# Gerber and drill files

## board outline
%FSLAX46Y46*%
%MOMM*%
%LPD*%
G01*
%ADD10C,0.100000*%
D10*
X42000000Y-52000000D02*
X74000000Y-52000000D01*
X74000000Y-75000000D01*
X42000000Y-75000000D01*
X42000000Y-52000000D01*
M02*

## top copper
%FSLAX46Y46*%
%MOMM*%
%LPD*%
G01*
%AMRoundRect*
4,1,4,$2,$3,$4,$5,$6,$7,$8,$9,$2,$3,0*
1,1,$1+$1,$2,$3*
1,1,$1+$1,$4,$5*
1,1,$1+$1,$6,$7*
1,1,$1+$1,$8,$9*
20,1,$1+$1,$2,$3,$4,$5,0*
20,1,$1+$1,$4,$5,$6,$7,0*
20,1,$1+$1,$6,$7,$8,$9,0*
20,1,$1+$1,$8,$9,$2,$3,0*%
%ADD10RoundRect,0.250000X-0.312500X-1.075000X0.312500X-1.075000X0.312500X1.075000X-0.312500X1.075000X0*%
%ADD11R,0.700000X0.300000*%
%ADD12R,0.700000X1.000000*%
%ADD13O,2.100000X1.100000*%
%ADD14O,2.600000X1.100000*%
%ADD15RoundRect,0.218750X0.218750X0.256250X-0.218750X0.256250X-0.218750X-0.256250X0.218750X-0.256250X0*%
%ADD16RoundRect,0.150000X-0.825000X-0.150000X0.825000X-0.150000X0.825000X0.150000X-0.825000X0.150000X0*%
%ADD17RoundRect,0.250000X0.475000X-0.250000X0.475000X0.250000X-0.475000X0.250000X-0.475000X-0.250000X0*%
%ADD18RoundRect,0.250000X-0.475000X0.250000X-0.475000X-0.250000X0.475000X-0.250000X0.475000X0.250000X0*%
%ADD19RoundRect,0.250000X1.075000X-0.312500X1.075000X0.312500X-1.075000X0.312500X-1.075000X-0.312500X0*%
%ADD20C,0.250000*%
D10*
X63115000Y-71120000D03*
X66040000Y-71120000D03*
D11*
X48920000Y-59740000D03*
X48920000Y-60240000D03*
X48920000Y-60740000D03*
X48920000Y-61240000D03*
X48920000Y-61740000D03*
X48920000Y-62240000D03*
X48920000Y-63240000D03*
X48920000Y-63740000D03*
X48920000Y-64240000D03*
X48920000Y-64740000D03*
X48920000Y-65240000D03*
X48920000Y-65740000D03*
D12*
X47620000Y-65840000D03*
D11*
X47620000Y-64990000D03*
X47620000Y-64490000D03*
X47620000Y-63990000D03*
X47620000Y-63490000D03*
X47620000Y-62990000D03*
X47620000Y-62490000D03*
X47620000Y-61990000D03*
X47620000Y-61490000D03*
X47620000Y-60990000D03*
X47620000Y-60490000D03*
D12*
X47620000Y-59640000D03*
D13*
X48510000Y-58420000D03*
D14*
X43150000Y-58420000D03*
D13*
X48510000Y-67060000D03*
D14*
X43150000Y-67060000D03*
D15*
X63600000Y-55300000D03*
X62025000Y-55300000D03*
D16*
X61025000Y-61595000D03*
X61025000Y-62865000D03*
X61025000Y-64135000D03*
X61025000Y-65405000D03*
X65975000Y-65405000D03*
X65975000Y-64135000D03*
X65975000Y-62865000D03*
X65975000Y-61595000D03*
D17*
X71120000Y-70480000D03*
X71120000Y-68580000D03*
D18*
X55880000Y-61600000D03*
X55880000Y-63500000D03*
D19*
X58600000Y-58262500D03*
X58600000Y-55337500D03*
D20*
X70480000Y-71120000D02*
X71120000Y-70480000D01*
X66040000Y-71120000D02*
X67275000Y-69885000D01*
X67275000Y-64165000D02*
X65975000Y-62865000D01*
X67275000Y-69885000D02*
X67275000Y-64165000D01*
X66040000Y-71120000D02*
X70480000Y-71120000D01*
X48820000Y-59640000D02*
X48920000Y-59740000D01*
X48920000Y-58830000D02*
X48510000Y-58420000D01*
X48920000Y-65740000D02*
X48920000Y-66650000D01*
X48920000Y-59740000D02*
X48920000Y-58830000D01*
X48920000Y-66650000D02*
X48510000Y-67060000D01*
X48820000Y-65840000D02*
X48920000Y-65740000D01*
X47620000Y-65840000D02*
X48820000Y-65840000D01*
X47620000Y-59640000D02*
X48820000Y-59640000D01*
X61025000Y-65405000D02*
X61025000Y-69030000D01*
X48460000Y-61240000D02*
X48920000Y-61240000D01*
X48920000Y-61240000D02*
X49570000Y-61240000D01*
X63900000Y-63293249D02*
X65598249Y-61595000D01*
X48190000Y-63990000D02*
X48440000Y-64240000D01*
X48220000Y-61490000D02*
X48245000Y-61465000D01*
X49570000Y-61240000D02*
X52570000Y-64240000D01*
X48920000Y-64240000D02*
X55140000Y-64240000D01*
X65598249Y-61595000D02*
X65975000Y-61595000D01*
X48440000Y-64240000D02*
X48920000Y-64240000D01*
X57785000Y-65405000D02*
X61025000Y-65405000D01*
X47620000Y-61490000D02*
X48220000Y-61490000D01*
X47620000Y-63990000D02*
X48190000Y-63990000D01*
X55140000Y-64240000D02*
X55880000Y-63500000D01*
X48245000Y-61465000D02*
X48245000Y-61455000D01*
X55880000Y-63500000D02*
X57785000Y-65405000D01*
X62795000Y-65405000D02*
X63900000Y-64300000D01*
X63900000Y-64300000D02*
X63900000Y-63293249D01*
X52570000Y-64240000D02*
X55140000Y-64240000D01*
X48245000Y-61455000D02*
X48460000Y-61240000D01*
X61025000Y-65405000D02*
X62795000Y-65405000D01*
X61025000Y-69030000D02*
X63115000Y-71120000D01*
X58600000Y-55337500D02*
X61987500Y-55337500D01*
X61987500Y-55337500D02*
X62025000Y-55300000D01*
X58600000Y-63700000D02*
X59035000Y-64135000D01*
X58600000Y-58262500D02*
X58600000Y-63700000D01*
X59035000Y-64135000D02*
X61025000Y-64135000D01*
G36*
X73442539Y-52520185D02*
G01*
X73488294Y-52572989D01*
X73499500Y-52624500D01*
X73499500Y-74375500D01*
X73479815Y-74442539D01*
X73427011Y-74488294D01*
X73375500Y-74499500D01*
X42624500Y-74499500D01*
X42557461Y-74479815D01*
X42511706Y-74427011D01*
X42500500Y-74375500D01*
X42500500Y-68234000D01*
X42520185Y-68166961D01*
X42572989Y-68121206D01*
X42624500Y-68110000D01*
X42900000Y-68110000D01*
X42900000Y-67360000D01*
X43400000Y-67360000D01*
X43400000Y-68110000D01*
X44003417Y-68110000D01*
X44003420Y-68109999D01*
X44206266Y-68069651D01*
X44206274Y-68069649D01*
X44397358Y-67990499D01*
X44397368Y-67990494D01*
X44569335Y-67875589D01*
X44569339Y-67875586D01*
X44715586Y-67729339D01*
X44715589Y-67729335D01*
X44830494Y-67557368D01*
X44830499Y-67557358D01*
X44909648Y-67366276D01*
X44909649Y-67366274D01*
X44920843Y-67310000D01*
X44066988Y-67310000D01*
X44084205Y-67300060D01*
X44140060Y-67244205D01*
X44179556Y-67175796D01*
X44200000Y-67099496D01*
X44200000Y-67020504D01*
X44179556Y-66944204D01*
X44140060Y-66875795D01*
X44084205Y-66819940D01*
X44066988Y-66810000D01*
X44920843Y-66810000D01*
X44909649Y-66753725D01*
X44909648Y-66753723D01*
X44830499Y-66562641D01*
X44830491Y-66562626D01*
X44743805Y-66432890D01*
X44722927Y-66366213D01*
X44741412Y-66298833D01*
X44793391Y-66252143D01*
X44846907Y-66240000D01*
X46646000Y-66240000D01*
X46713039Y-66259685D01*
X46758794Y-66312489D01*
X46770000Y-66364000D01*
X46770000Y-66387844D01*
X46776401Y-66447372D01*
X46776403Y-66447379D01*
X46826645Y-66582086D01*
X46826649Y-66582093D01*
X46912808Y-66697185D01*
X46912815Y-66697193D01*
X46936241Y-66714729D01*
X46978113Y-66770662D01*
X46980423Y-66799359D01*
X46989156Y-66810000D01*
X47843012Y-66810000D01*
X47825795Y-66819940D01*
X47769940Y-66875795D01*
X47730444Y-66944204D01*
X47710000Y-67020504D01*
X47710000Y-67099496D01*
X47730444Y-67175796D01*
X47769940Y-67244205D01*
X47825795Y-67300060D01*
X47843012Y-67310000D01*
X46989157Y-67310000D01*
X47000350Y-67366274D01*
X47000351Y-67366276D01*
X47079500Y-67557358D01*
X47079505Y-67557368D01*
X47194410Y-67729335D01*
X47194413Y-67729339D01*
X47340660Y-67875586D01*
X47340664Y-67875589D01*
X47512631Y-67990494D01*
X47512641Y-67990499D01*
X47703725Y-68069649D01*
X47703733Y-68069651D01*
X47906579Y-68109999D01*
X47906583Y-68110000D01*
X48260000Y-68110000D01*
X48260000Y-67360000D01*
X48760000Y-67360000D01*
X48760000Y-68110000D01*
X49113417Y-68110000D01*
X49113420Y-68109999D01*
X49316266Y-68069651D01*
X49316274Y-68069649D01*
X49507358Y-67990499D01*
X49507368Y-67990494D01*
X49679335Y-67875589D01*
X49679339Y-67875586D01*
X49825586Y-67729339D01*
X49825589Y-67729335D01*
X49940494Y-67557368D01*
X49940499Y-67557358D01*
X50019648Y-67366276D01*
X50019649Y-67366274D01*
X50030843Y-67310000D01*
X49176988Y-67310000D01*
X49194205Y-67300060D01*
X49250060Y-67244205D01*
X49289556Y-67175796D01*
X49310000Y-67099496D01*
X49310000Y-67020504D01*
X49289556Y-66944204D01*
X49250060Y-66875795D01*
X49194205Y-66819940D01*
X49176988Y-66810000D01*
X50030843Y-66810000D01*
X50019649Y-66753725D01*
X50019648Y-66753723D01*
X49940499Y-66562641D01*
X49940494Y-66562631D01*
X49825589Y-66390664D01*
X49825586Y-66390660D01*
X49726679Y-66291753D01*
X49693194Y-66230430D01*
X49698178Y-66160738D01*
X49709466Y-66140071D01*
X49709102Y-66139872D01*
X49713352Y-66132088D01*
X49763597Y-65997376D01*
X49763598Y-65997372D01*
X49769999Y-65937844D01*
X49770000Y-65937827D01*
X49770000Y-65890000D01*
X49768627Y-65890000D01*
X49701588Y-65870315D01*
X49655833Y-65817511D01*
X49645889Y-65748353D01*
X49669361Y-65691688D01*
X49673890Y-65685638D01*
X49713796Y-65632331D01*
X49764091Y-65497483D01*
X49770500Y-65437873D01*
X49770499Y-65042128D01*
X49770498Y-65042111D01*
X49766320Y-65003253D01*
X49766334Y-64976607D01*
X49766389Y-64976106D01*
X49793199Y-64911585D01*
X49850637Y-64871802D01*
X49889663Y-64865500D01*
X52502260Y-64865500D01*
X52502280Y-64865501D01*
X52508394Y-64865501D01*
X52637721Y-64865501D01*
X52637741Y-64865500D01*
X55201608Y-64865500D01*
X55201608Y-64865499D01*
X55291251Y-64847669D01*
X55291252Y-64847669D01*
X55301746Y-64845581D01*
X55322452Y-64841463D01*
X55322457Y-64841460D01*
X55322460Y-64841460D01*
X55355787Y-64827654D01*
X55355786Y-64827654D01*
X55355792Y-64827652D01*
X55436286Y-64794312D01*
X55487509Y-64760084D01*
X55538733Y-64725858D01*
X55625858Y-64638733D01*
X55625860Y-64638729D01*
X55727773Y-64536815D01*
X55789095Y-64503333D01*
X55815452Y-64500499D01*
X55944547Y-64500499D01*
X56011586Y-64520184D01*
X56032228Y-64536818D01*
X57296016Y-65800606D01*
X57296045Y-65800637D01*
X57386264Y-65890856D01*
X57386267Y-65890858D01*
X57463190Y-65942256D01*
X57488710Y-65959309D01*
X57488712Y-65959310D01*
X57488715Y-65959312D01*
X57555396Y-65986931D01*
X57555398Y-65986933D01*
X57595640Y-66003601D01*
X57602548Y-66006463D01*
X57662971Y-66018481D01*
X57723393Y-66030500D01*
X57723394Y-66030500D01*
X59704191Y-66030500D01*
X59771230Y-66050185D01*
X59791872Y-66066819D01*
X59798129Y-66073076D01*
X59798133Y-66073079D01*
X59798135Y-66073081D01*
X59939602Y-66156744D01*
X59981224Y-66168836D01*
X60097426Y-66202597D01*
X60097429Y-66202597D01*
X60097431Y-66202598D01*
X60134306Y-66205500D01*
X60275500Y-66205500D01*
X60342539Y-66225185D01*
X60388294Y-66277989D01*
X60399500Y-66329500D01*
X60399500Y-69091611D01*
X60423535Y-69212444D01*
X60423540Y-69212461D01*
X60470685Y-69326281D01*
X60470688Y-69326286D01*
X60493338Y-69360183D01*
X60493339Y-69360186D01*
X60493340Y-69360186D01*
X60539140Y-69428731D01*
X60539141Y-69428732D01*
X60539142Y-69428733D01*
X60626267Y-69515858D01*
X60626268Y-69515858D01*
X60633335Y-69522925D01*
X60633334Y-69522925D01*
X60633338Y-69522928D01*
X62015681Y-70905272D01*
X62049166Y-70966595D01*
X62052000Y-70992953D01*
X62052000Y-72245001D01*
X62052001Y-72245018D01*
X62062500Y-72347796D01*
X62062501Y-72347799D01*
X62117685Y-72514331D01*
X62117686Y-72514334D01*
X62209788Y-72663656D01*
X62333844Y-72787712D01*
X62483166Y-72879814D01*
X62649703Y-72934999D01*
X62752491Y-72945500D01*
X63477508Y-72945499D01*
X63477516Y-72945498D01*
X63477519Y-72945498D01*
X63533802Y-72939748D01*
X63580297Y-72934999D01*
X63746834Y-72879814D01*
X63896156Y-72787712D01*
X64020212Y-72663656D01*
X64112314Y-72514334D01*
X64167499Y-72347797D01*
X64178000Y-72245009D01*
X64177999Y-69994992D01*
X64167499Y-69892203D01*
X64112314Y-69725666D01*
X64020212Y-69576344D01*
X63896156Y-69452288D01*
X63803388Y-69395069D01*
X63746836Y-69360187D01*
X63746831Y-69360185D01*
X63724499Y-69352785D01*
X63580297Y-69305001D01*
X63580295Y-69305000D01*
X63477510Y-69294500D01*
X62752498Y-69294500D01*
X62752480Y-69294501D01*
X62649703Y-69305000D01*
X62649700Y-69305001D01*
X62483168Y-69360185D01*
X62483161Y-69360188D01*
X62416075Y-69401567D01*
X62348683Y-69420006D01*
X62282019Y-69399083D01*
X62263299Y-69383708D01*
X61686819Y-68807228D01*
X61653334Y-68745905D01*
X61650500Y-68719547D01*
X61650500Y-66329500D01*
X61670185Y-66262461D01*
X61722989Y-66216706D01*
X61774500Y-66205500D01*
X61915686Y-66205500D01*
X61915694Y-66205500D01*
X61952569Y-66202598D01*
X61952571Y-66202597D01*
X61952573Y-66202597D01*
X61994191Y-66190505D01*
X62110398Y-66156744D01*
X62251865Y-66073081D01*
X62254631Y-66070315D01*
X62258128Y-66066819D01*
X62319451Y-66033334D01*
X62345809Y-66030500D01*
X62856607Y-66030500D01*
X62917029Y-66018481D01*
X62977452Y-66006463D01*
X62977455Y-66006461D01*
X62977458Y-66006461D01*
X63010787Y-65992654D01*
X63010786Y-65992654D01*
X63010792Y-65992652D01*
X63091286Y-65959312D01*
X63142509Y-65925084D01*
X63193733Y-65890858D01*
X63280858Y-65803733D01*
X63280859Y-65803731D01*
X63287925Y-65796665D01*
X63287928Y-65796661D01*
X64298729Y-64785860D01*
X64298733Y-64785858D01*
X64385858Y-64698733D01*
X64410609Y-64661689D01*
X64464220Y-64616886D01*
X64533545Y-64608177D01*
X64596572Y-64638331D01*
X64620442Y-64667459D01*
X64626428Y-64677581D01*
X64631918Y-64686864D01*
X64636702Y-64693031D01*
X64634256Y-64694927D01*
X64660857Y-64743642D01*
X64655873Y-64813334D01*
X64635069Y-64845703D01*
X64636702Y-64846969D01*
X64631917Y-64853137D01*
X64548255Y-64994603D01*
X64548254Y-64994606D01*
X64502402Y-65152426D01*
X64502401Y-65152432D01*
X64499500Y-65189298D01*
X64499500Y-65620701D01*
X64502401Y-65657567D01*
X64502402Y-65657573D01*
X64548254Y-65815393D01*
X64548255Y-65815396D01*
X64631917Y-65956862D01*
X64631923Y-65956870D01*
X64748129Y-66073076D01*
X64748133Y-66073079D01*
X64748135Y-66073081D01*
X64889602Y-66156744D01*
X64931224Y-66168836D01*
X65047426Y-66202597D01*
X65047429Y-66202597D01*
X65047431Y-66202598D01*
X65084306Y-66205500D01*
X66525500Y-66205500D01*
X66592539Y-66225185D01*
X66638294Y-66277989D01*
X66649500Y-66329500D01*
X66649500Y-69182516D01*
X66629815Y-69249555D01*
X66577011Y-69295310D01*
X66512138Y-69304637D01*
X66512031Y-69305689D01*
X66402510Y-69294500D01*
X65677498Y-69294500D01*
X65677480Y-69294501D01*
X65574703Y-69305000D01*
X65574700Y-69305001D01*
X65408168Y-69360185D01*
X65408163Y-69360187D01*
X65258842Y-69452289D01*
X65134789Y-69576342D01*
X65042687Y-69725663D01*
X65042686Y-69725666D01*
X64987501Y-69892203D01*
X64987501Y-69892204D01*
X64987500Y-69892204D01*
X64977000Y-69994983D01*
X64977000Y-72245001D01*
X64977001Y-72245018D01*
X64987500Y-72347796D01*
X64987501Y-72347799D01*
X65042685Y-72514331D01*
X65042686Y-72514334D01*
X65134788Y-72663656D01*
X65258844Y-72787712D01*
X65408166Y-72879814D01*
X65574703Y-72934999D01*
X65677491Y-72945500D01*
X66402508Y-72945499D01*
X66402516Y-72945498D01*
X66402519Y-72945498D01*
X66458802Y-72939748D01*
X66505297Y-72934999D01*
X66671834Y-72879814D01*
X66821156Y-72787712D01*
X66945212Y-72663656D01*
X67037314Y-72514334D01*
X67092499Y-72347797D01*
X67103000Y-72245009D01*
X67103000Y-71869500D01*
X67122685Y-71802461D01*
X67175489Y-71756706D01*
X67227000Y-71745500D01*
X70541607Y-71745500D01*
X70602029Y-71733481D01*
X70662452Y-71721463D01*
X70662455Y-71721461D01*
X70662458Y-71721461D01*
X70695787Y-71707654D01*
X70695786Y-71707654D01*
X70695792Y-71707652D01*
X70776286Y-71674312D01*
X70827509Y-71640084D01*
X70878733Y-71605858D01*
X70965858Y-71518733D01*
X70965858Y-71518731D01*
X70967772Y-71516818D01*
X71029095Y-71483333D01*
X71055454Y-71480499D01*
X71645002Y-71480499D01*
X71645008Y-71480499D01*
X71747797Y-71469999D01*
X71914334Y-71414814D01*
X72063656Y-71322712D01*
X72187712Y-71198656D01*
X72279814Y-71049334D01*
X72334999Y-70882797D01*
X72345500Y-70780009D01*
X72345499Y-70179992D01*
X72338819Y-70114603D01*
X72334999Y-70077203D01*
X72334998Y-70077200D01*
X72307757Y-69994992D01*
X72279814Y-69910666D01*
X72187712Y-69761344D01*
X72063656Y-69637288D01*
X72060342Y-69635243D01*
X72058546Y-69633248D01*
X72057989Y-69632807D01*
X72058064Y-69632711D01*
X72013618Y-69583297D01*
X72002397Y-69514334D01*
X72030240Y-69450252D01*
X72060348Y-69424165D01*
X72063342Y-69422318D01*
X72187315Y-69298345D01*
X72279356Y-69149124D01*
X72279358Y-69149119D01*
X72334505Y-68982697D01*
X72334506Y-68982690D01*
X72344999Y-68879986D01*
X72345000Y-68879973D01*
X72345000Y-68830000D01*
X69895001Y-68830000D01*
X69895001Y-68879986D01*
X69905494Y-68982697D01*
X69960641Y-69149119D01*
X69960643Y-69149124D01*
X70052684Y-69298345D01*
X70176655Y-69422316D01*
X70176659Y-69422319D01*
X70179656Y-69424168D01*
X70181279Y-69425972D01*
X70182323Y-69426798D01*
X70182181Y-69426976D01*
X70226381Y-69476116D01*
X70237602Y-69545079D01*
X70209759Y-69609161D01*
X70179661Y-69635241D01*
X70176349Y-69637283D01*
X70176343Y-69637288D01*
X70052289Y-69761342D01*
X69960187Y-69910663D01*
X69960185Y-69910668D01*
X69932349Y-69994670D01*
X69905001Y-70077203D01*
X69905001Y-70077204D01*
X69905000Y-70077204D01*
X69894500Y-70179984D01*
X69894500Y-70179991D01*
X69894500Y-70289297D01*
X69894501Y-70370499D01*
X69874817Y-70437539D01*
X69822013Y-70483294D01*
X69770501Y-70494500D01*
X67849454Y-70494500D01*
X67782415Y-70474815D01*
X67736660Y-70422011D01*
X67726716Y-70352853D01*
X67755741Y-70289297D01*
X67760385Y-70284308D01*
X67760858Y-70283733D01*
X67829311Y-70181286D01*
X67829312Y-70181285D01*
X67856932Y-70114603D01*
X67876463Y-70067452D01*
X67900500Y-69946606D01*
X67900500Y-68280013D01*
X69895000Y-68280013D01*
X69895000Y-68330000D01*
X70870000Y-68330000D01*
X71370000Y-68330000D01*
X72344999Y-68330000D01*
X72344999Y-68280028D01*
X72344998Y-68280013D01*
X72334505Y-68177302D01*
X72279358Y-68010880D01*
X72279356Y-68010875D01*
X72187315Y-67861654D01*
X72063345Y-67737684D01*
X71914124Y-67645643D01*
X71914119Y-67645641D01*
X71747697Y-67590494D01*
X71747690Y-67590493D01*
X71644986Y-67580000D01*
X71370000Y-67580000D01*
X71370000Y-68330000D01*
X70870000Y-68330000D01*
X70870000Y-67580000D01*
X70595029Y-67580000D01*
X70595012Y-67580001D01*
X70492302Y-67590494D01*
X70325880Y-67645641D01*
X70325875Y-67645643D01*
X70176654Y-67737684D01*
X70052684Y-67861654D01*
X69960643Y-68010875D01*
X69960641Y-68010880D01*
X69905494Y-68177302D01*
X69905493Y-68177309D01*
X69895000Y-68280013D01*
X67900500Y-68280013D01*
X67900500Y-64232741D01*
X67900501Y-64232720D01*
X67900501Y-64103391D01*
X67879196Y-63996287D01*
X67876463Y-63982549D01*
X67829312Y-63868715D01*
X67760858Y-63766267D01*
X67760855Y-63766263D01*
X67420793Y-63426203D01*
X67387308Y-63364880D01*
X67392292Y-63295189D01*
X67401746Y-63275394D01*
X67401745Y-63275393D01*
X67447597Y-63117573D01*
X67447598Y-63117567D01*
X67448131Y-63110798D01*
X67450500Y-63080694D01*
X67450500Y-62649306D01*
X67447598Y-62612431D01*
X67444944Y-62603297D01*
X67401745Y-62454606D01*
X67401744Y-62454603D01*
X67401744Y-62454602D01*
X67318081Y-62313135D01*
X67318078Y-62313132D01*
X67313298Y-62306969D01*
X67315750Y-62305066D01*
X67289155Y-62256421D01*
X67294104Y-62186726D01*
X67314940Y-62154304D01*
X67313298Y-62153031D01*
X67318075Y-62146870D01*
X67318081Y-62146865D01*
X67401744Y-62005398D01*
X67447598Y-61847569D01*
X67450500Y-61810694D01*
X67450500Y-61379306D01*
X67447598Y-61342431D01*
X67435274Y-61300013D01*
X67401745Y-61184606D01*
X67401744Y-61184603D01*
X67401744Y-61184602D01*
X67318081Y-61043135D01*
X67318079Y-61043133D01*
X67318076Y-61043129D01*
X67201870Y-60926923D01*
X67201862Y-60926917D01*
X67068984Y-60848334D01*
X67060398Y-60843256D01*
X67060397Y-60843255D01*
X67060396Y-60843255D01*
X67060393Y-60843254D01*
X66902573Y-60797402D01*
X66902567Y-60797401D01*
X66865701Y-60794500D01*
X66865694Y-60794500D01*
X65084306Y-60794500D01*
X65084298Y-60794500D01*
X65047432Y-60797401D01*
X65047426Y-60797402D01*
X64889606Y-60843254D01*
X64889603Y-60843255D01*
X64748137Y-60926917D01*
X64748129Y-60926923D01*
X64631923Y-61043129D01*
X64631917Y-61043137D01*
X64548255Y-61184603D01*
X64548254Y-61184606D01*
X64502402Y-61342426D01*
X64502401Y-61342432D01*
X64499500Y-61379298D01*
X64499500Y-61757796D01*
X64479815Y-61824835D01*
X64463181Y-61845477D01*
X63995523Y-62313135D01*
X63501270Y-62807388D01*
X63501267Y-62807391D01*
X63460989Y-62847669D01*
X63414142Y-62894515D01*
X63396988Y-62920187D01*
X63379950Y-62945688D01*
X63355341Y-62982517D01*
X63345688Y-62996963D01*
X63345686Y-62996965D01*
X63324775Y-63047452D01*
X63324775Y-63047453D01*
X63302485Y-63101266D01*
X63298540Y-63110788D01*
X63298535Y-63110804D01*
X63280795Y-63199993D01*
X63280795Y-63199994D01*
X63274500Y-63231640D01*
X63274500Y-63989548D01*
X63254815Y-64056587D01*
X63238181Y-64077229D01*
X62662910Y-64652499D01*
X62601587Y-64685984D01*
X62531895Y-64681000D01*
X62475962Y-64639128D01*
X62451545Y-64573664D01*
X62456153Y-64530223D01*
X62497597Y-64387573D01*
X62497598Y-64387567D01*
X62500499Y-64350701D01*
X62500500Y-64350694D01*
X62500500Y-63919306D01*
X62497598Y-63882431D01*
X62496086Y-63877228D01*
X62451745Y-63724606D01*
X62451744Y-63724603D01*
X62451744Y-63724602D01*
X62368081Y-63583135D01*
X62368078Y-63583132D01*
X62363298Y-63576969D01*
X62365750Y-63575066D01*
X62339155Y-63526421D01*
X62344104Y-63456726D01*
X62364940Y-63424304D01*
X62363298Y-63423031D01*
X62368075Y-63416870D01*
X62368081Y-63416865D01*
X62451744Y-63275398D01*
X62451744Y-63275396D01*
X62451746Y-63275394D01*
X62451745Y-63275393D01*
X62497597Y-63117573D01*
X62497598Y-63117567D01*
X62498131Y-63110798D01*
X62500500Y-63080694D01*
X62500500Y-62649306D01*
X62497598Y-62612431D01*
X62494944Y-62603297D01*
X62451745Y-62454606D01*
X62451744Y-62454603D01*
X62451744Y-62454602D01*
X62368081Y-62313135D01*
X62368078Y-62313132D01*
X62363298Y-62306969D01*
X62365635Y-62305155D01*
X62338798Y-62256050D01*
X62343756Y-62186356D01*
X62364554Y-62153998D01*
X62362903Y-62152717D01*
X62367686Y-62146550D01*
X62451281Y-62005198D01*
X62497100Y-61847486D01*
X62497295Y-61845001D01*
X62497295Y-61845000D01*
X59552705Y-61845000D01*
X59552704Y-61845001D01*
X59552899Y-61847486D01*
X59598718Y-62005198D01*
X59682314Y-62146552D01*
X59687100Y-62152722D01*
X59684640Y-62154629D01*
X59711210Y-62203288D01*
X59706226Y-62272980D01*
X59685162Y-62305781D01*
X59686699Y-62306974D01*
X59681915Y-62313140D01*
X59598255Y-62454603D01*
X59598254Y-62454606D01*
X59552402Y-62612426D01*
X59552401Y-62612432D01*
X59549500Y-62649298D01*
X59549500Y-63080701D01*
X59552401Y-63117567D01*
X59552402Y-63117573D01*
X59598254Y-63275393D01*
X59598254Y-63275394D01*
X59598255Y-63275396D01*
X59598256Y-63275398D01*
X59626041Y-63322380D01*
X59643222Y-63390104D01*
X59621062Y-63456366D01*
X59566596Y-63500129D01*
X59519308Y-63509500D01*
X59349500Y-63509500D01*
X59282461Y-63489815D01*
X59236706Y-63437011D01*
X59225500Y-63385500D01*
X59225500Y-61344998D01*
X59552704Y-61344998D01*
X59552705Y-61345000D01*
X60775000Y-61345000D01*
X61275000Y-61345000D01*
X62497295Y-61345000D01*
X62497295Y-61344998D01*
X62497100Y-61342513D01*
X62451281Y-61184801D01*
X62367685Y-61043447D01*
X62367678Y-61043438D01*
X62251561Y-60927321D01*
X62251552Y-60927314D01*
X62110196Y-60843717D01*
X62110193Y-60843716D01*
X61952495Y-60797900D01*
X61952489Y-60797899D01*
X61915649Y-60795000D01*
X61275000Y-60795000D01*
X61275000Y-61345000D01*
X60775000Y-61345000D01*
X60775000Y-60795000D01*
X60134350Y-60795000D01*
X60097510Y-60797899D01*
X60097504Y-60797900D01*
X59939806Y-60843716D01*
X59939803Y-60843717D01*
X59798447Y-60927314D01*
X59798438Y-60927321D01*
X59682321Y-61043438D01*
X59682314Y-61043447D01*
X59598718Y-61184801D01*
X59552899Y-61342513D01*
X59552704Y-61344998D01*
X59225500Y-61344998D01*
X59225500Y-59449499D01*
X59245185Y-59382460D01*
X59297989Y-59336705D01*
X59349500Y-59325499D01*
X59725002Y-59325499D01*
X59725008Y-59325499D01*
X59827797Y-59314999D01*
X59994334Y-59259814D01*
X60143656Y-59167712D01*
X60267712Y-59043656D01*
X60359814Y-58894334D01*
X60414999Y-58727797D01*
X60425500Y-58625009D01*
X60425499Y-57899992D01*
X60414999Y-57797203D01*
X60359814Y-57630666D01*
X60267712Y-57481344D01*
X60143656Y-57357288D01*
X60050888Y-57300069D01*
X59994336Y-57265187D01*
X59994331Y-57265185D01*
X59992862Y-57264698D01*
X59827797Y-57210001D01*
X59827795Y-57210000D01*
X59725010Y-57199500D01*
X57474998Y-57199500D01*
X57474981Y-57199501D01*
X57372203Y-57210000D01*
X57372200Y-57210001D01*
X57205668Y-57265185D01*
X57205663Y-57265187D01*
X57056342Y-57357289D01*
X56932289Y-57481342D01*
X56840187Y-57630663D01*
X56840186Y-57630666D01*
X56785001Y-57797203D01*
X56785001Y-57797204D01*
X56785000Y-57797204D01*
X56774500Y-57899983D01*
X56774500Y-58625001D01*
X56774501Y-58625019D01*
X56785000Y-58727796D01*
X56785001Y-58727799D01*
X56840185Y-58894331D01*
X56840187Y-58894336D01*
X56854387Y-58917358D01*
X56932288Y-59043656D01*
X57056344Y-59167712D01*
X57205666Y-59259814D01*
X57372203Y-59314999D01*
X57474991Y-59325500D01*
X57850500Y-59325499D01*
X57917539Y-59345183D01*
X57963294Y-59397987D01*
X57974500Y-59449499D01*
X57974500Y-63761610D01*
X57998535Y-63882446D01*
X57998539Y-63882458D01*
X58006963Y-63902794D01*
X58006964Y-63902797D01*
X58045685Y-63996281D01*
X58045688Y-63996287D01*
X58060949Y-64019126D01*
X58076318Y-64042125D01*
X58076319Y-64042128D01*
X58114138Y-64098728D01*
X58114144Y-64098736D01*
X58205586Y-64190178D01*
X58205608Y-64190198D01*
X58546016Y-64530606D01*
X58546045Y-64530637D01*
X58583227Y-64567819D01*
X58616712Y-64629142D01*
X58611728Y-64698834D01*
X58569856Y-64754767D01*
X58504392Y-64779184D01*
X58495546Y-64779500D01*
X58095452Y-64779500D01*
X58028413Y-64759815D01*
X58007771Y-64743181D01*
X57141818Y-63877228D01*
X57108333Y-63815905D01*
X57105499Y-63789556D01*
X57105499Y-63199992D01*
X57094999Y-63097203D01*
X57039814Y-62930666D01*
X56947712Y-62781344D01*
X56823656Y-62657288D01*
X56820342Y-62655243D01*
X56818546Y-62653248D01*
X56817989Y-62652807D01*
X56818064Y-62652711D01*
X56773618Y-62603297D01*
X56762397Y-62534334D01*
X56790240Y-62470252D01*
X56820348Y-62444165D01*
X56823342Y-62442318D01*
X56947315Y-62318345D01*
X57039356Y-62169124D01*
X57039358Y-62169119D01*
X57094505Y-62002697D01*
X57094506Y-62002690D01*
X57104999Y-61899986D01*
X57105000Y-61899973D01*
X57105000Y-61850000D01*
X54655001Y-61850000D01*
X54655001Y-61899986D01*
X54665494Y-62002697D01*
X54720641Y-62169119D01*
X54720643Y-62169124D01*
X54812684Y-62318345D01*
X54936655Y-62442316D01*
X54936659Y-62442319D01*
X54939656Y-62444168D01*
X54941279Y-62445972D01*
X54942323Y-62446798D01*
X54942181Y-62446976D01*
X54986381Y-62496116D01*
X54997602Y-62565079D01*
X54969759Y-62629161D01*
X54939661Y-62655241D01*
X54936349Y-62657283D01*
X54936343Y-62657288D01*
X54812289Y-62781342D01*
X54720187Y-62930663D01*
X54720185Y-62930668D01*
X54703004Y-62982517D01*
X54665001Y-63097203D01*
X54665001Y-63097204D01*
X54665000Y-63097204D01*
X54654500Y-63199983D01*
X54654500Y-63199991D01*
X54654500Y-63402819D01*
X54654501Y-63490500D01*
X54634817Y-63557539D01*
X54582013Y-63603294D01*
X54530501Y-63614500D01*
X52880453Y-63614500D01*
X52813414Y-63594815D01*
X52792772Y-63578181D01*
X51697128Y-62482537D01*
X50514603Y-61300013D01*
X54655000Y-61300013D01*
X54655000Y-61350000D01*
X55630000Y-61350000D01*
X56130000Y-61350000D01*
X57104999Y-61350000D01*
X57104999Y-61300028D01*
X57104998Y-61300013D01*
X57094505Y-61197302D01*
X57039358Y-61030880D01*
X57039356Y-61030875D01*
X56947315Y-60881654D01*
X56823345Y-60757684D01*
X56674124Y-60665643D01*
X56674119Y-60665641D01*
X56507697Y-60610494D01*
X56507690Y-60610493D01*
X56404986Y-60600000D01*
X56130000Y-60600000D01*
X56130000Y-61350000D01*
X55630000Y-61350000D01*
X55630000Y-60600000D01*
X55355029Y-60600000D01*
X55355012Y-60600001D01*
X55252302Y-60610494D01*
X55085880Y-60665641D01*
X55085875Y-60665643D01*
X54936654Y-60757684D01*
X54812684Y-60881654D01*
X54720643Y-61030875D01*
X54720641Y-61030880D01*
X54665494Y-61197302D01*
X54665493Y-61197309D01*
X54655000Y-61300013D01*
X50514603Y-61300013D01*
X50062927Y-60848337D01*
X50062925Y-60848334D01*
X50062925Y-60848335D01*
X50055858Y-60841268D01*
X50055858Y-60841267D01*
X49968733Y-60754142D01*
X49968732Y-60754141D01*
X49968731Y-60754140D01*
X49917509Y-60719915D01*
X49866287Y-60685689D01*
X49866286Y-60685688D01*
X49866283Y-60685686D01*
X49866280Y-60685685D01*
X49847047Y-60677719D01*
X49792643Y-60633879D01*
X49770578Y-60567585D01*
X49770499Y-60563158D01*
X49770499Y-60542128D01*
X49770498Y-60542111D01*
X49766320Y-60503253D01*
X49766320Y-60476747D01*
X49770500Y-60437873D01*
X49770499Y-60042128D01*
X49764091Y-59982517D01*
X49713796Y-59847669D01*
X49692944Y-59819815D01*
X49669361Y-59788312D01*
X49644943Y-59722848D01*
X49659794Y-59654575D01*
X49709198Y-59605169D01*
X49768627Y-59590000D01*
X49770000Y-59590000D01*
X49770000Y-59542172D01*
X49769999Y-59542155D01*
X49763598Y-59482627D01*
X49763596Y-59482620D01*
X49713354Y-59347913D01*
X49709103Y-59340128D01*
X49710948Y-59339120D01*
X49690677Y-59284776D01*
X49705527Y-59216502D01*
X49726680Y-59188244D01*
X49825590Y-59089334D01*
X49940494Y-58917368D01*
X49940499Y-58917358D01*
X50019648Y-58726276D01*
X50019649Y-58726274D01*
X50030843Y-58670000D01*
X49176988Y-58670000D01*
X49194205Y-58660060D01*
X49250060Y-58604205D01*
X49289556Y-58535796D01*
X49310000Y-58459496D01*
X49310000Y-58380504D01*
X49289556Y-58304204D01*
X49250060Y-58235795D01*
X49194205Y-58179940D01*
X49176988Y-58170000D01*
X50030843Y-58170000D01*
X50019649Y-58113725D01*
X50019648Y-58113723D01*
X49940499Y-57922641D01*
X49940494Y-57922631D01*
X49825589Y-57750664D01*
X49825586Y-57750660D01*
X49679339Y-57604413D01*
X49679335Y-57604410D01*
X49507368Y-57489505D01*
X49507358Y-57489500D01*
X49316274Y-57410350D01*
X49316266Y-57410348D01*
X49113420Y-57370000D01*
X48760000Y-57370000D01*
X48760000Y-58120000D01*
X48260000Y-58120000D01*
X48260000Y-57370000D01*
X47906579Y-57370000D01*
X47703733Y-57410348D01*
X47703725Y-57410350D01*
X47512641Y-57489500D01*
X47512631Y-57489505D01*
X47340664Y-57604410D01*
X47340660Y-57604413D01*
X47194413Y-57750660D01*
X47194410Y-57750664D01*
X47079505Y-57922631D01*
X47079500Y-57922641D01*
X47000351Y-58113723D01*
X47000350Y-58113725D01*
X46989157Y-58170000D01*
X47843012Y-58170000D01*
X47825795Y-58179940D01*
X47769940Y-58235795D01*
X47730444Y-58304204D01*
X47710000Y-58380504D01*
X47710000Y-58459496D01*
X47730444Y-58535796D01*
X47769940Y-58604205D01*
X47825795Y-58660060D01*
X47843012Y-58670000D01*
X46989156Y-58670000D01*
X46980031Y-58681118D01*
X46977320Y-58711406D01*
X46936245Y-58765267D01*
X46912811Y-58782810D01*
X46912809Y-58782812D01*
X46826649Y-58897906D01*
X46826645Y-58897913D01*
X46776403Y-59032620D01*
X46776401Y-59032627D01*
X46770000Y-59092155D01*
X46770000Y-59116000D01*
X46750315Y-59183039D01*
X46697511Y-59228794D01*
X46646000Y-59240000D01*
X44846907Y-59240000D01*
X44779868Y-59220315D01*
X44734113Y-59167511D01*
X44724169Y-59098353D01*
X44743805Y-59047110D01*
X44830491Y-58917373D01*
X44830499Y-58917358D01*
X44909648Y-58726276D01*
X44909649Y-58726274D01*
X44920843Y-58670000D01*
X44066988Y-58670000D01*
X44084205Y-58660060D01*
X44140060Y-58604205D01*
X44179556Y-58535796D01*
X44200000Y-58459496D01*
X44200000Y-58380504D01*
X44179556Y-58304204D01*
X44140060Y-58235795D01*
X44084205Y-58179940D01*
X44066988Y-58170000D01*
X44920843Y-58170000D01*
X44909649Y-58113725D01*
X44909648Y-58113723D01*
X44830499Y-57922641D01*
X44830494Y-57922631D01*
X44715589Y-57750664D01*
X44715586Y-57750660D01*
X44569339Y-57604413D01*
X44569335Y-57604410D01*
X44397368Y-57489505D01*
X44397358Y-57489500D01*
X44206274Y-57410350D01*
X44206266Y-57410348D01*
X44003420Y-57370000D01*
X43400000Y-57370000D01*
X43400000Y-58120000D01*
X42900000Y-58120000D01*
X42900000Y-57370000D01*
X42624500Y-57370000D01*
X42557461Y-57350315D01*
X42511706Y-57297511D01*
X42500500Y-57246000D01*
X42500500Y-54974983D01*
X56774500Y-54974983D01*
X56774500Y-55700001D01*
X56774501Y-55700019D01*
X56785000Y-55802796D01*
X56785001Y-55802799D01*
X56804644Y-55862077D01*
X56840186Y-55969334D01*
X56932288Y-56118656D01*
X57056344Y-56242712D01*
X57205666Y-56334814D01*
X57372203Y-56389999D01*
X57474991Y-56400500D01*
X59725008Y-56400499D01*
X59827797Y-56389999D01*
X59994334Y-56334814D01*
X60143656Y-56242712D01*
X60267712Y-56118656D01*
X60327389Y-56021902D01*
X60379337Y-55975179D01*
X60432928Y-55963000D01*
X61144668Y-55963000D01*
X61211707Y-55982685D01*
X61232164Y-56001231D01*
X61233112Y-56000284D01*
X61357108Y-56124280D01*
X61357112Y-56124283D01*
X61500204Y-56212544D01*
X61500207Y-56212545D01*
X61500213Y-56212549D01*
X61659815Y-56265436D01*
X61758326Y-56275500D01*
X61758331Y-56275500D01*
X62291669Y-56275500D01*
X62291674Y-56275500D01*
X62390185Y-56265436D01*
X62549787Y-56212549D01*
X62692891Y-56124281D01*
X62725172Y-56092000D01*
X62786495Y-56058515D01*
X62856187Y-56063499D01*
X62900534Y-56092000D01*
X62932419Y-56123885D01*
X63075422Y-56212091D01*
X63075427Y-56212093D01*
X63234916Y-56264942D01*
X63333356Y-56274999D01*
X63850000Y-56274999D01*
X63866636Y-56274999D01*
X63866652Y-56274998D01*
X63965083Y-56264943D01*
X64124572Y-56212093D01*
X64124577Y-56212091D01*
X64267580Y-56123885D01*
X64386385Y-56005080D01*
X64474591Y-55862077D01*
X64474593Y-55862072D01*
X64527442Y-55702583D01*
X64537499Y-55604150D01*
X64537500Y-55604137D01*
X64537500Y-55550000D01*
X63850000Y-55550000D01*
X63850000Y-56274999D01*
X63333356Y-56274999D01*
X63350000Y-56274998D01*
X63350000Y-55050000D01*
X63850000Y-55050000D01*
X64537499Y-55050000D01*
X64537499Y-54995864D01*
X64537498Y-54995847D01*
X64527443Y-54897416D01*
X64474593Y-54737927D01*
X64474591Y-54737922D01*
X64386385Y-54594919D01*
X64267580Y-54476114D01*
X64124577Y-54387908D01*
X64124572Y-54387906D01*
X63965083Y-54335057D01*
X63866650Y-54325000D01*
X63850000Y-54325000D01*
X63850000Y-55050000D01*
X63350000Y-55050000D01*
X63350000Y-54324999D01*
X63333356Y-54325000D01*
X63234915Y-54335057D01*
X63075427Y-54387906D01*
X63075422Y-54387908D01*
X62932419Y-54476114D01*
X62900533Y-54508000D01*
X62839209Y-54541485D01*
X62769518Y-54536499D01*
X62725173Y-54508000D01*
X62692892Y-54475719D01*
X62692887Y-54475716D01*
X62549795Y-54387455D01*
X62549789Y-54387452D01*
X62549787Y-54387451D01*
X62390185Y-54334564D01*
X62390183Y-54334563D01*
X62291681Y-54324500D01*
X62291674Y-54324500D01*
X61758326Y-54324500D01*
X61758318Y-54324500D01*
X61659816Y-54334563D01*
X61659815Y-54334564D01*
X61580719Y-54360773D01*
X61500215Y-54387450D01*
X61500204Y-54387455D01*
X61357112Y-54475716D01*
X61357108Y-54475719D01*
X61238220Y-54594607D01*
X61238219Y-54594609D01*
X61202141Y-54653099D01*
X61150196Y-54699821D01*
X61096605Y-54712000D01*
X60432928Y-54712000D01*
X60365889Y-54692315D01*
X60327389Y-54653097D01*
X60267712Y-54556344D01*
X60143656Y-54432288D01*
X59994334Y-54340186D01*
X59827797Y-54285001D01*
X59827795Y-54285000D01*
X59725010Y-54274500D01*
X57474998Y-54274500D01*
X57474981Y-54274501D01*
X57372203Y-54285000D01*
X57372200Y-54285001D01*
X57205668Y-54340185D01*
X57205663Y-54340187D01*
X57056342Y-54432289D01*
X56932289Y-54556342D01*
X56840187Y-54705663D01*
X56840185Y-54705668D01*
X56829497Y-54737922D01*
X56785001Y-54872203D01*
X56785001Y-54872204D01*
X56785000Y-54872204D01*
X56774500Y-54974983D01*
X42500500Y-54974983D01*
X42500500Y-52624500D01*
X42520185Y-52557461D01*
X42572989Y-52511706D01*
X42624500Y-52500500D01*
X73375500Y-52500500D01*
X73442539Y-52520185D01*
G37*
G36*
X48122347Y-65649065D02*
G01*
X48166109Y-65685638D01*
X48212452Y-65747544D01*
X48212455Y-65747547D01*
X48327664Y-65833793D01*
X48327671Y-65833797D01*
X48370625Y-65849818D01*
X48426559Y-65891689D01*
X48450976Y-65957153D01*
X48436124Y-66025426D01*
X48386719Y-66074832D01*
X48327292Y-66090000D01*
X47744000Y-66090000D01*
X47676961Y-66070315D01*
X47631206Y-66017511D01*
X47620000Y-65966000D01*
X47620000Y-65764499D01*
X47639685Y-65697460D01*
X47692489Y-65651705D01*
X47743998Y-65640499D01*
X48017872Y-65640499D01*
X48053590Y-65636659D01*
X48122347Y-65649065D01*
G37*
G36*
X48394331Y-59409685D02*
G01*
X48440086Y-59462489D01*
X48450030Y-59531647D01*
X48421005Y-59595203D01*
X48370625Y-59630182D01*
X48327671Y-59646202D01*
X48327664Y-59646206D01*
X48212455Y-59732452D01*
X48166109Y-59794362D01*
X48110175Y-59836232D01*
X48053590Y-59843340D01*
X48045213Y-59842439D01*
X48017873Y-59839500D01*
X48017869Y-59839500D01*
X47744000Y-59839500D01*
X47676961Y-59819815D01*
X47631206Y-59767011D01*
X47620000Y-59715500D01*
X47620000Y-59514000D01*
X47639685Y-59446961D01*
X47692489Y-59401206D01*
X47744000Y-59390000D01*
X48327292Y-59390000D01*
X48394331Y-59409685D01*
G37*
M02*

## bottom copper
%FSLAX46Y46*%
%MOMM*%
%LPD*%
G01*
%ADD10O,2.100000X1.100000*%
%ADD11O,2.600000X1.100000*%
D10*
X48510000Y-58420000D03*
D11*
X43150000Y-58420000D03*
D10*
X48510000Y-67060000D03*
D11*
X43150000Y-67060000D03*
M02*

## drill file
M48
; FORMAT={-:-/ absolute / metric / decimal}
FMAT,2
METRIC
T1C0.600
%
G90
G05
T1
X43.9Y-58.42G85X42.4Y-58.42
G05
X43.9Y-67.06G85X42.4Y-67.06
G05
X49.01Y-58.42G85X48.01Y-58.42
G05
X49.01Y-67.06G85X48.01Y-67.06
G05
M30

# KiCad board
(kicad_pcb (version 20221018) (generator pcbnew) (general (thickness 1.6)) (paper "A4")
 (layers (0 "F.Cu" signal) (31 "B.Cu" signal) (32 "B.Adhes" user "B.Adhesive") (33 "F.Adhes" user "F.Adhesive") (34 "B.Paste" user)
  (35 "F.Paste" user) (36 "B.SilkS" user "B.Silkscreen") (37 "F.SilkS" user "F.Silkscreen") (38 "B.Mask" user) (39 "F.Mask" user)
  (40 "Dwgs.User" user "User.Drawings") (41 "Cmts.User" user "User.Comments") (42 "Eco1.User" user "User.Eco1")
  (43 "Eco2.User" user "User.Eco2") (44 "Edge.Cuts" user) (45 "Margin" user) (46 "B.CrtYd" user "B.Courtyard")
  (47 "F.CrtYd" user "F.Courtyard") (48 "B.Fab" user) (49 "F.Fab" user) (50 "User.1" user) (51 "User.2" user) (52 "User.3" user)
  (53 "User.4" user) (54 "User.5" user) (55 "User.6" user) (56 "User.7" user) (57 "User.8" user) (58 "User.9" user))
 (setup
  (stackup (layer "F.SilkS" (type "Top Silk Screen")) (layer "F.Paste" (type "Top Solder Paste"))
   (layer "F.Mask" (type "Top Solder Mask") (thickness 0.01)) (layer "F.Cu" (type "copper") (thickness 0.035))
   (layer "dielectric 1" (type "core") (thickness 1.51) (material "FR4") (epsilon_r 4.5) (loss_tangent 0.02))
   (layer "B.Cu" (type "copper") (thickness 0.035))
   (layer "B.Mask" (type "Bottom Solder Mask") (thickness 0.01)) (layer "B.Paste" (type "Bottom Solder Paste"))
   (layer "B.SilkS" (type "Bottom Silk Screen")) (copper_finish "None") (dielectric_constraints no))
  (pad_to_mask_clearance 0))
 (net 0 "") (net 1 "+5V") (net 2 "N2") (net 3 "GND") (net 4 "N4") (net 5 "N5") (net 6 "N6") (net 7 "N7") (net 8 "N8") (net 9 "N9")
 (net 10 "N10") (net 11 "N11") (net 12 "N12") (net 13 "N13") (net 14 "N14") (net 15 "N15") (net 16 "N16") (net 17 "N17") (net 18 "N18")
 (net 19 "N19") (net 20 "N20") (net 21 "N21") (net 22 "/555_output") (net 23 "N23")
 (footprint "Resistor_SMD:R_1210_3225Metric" (layer "F.Cu") (at 64.5775 71.12)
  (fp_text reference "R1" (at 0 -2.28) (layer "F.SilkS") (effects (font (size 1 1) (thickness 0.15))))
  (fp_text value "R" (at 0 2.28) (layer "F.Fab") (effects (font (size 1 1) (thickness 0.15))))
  (pad "1" smd roundrect (at -1.4625 0) (size 1.125 2.65) (layers "F.Cu" "F.Paste" "F.Mask") (roundrect_rratio 0.222222) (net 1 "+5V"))
  (pad "2" smd roundrect (at 1.4625 0) (size 1.125 2.65) (layers "F.Cu" "F.Paste" "F.Mask") (roundrect_rratio 0.222222) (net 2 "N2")))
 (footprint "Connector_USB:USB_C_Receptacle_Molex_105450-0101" (layer "F.Cu") (at 45.705 62.74 -90)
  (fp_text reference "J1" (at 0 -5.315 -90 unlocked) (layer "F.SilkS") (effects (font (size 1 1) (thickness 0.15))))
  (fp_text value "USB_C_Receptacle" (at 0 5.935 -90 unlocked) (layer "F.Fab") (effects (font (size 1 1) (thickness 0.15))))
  (pad "A1" smd rect (at -3 -3.215 270) (size 0.3 0.7) (layers "F.Cu" "F.Paste" "F.Mask") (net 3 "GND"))
  (pad "A2" smd rect (at -2.5 -3.215 270) (size 0.3 0.7) (layers "F.Cu" "F.Paste" "F.Mask") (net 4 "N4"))
  (pad "A3" smd rect (at -2 -3.215 270) (size 0.3 0.7) (layers "F.Cu" "F.Paste" "F.Mask") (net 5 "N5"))
  (pad "A4" smd rect (at -1.5 -3.215 270) (size 0.3 0.7) (layers "F.Cu" "F.Paste" "F.Mask") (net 1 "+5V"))
  (pad "A5" smd rect (at -1 -3.215 270) (size 0.3 0.7) (layers "F.Cu" "F.Paste" "F.Mask") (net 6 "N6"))
  (pad "A6" smd rect (at -0.5 -3.215 270) (size 0.3 0.7) (layers "F.Cu" "F.Paste" "F.Mask") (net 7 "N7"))
  (pad "A7" smd rect (at 0.5 -3.215 270) (size 0.3 0.7) (layers "F.Cu" "F.Paste" "F.Mask") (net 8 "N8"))
  (pad "A8" smd rect (at 1 -3.215 270) (size 0.3 0.7) (layers "F.Cu" "F.Paste" "F.Mask") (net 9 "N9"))
  (pad "A9" smd rect (at 1.5 -3.215 270) (size 0.3 0.7) (layers "F.Cu" "F.Paste" "F.Mask") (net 1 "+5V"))
  (pad "A10" smd rect (at 2 -3.215 270) (size 0.3 0.7) (layers "F.Cu" "F.Paste" "F.Mask") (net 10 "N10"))
  (pad "A11" smd rect (at 2.5 -3.215 270) (size 0.3 0.7) (layers "F.Cu" "F.Paste" "F.Mask") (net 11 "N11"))
  (pad "A12" smd rect (at 3 -3.215 270) (size 0.3 0.7) (layers "F.Cu" "F.Paste" "F.Mask") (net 3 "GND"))
  (pad "B1" smd rect (at 3.1 -1.915 270) (size 1 0.7) (layers "F.Cu" "F.Paste" "F.Mask") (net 3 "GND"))
  (pad "B2" smd rect (at 2.25 -1.915 270) (size 0.3 0.7) (layers "F.Cu" "F.Paste" "F.Mask") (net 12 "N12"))
  (pad "B3" smd rect (at 1.75 -1.915 270) (size 0.3 0.7) (layers "F.Cu" "F.Paste" "F.Mask") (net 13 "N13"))
  (pad "B4" smd rect (at 1.25 -1.915 270) (size 0.3 0.7) (layers "F.Cu" "F.Paste" "F.Mask") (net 1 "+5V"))
  (pad "B5" smd rect (at 0.75 -1.915 270) (size 0.3 0.7) (layers "F.Cu" "F.Paste" "F.Mask") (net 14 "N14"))
  (pad "B6" smd rect (at 0.25 -1.915 270) (size 0.3 0.7) (layers "F.Cu" "F.Paste" "F.Mask") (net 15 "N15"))
  (pad "B7" smd rect (at -0.25 -1.915 270) (size 0.3 0.7) (layers "F.Cu" "F.Paste" "F.Mask") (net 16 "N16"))
  (pad "B8" smd rect (at -0.75 -1.915 270) (size 0.3 0.7) (layers "F.Cu" "F.Paste" "F.Mask") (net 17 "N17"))
  (pad "B9" smd rect (at -1.25 -1.915 270) (size 0.3 0.7) (layers "F.Cu" "F.Paste" "F.Mask") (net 1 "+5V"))
  (pad "B10" smd rect (at -1.75 -1.915 270) (size 0.3 0.7) (layers "F.Cu" "F.Paste" "F.Mask") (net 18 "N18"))
  (pad "B11" smd rect (at -2.25 -1.915 270) (size 0.3 0.7) (layers "F.Cu" "F.Paste" "F.Mask") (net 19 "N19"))
  (pad "B12" smd rect (at -3.1 -1.915 270) (size 1 0.7) (layers "F.Cu" "F.Paste" "F.Mask") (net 3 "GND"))
  (pad "S1" thru_hole oval (at -4.32 -2.805 270) (size 1.1 2.1) (drill oval 0.6 1.6) (layers "*.Cu" "*.Mask") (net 3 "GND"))
  (pad "S1" thru_hole oval (at -4.32 2.555 270) (size 1.1 2.6) (drill oval 0.6 2.1) (layers "*.Cu" "*.Mask") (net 3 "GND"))
  (pad "S1" thru_hole oval (at 4.32 -2.805 270) (size 1.1 2.1) (drill oval 0.6 1.6) (layers "*.Cu" "*.Mask") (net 3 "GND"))
  (pad "S1" thru_hole oval (at 4.32 2.555 270) (size 1.1 2.6) (drill oval 0.6 2.1) (layers "*.Cu" "*.Mask") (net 3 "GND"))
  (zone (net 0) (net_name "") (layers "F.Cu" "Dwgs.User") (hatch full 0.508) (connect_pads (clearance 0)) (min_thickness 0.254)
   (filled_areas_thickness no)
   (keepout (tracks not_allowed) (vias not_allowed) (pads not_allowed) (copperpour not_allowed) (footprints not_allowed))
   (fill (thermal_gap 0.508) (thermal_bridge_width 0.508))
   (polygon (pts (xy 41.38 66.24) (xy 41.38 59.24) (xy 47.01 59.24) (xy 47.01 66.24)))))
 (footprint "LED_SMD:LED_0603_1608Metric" (layer "F.Cu") (at 62.8125 55.3 180)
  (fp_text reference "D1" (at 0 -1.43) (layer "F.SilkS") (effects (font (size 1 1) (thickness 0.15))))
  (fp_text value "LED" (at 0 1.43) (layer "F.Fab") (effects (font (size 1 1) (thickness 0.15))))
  (pad "1" smd roundrect (at -0.7875 0 180) (size 0.875 0.95) (layers "F.Cu" "F.Paste" "F.Mask") (roundrect_rratio 0.25) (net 3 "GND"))
  (pad "2" smd roundrect (at 0.7875 0 180) (size 0.875 0.95) (layers "F.Cu" "F.Paste" "F.Mask") (roundrect_rratio 0.25) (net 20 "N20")))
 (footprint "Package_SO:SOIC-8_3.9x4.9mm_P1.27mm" (layer "F.Cu") (at 63.5 63.5)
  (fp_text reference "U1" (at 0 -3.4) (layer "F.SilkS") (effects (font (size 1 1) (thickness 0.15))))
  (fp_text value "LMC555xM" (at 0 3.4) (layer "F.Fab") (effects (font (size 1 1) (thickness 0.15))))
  (pad "1" smd roundrect (at -2.475 -1.905) (size 1.95 0.6) (layers "F.Cu" "F.Paste" "F.Mask") (roundrect_rratio 0.25) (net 3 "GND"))
  (pad "2" smd roundrect (at -2.475 -0.635) (size 1.95 0.6) (layers "F.Cu" "F.Paste" "F.Mask") (roundrect_rratio 0.25) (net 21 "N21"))
  (pad "3" smd roundrect (at -2.475 0.635) (size 1.95 0.6) (layers "F.Cu" "F.Paste" "F.Mask") (roundrect_rratio 0.25) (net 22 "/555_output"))
  (pad "4" smd roundrect (at -2.475 1.905) (size 1.95 0.6) (layers "F.Cu" "F.Paste" "F.Mask") (roundrect_rratio 0.25) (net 1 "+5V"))
  (pad "5" smd roundrect (at 2.475 1.905) (size 1.95 0.6) (layers "F.Cu" "F.Paste" "F.Mask") (roundrect_rratio 0.25) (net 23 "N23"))
  (pad "6" smd roundrect (at 2.475 0.635) (size 1.95 0.6) (layers "F.Cu" "F.Paste" "F.Mask") (roundrect_rratio 0.25) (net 2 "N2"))
  (pad "7" smd roundrect (at 2.475 -0.635) (size 1.95 0.6) (layers "F.Cu" "F.Paste" "F.Mask") (roundrect_rratio 0.25) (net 2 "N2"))
  (pad "8" smd roundrect (at 2.475 -1.905) (size 1.95 0.6) (layers "F.Cu" "F.Paste" "F.Mask") (roundrect_rratio 0.25) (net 1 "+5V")))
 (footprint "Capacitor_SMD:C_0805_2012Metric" (layer "F.Cu") (at 71.12 69.53 90)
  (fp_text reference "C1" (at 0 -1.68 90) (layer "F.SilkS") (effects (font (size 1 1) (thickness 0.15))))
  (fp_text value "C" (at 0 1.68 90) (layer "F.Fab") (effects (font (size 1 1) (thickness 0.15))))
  (pad "1" smd roundrect (at -0.95 0 90) (size 1 1.45) (layers "F.Cu" "F.Paste" "F.Mask") (roundrect_rratio 0.25) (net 2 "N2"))
  (pad "2" smd roundrect (at 0.95 0 90) (size 1 1.45) (layers "F.Cu" "F.Paste" "F.Mask") (roundrect_rratio 0.25) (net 3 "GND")))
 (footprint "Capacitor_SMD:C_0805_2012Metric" (layer "F.Cu") (at 55.88 62.55 -90)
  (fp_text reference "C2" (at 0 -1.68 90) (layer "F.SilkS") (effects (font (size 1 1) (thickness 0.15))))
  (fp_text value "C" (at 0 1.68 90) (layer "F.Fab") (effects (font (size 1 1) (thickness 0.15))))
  (pad "1" smd roundrect (at -0.95 0 270) (size 1 1.45) (layers "F.Cu" "F.Paste" "F.Mask") (roundrect_rratio 0.25) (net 3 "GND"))
  (pad "2" smd roundrect (at 0.95 0 270) (size 1 1.45) (layers "F.Cu" "F.Paste" "F.Mask") (roundrect_rratio 0.25) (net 1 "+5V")))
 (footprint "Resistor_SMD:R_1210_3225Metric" (layer "F.Cu") (at 58.6 56.8 90)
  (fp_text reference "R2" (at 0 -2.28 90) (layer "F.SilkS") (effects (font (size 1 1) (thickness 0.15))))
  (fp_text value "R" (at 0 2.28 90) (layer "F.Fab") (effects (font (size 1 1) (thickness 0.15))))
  (pad "1" smd roundrect (at -1.4625 0 90) (size 1.125 2.65) (layers "F.Cu" "F.Paste" "F.Mask") (roundrect_rratio 0.222222)
   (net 22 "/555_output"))
  (pad "2" smd roundrect (at 1.4625 0 90) (size 1.125 2.65) (layers "F.Cu" "F.Paste" "F.Mask") (roundrect_rratio 0.222222) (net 20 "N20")))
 (gr_rect (start 42 52) (end 74 75) (stroke (width 0.1) (type default)) (fill none) (layer "Edge.Cuts"))
 (segment (start 70.48 71.12) (end 71.12 70.48) (width 0.25) (layer "F.Cu") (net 2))
 (segment (start 66.04 71.12) (end 67.275 69.885) (width 0.25) (layer "F.Cu") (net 2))
 (segment (start 67.275 64.165) (end 65.975 62.865) (width 0.25) (layer "F.Cu") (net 2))
 (segment (start 67.275 69.885) (end 67.275 64.165) (width 0.25) (layer "F.Cu") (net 2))
 (segment (start 66.04 71.12) (end 70.48 71.12) (width 0.25) (layer "F.Cu") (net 2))
 (segment (start 48.82 59.64) (end 48.92 59.74) (width 0.25) (layer "F.Cu") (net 3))
 (segment (start 48.92 58.83) (end 48.51 58.42) (width 0.25) (layer "F.Cu") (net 3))
 (segment (start 48.92 65.74) (end 48.92 66.65) (width 0.25) (layer "F.Cu") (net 3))
 (segment (start 48.92 59.74) (end 48.92 58.83) (width 0.25) (layer "F.Cu") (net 3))
 (segment (start 48.92 66.65) (end 48.51 67.06) (width 0.25) (layer "F.Cu") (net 3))
 (segment (start 48.82 65.84) (end 48.92 65.74) (width 0.25) (layer "F.Cu") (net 3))
 (segment (start 47.62 65.84) (end 48.82 65.84) (width 0.25) (layer "F.Cu") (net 3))
 (segment (start 47.62 59.64) (end 48.82 59.64) (width 0.25) (layer "F.Cu") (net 3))
 (segment (start 61.025 65.405) (end 61.025 69.03) (width 0.25) (layer "F.Cu") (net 1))
 (segment (start 48.46 61.24) (end 48.92 61.24) (width 0.25) (layer "F.Cu") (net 1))
 (segment (start 48.92 61.24) (end 49.57 61.24) (width 0.25) (layer "F.Cu") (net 1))
 (segment (start 63.9 63.293249) (end 65.598249 61.595) (width 0.25) (layer "F.Cu") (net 1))
 (segment (start 48.19 63.99) (end 48.44 64.24) (width 0.25) (layer "F.Cu") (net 1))
 (segment (start 48.22 61.49) (end 48.245 61.465) (width 0.25) (layer "F.Cu") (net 1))
 (segment (start 49.57 61.24) (end 52.57 64.24) (width 0.25) (layer "F.Cu") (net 1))
 (segment (start 48.92 64.24) (end 55.14 64.24) (width 0.25) (layer "F.Cu") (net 1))
 (segment (start 65.598249 61.595) (end 65.975 61.595) (width 0.25) (layer "F.Cu") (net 1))
 (segment (start 48.44 64.24) (end 48.92 64.24) (width 0.25) (layer "F.Cu") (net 1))
 (segment (start 57.785 65.405) (end 61.025 65.405) (width 0.25) (layer "F.Cu") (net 1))
 (segment (start 47.62 61.49) (end 48.22 61.49) (width 0.25) (layer "F.Cu") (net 1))
 (segment (start 47.62 63.99) (end 48.19 63.99) (width 0.25) (layer "F.Cu") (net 1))
 (segment (start 55.14 64.24) (end 55.88 63.5) (width 0.25) (layer "F.Cu") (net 1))
 (segment (start 48.245 61.465) (end 48.245 61.455) (width 0.25) (layer "F.Cu") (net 1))
 (segment (start 55.88 63.5) (end 57.785 65.405) (width 0.25) (layer "F.Cu") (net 1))
 (segment (start 62.795 65.405) (end 63.9 64.3) (width 0.25) (layer "F.Cu") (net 1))
 (segment (start 63.9 64.3) (end 63.9 63.293249) (width 0.25) (layer "F.Cu") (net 1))
 (segment (start 52.57 64.24) (end 55.14 64.24) (width 0.25) (layer "F.Cu") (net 1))
 (segment (start 48.245 61.455) (end 48.46 61.24) (width 0.25) (layer "F.Cu") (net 1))
 (segment (start 61.025 65.405) (end 62.795 65.405) (width 0.25) (layer "F.Cu") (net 1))
 (segment (start 61.025 69.03) (end 63.115 71.12) (width 0.25) (layer "F.Cu") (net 1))
 (segment (start 58.6 55.3375) (end 61.9875 55.3375) (width 0.25) (layer "F.Cu") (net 20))
 (segment (start 61.9875 55.3375) (end 62.025 55.3) (width 0.25) (layer "F.Cu") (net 20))
 (segment (start 58.6 63.7) (end 59.035 64.135) (width 0.25) (layer "F.Cu") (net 22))
 (segment (start 58.6 58.2625) (end 58.6 63.7) (width 0.25) (layer "F.Cu") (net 22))
 (segment (start 59.035 64.135) (end 61.025 64.135) (width 0.25) (layer "F.Cu") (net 22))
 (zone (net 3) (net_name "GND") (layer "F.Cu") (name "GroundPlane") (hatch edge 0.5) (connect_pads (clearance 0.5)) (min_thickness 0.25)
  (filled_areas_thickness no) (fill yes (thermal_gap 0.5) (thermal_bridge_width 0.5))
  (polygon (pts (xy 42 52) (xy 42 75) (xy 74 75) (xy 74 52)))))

